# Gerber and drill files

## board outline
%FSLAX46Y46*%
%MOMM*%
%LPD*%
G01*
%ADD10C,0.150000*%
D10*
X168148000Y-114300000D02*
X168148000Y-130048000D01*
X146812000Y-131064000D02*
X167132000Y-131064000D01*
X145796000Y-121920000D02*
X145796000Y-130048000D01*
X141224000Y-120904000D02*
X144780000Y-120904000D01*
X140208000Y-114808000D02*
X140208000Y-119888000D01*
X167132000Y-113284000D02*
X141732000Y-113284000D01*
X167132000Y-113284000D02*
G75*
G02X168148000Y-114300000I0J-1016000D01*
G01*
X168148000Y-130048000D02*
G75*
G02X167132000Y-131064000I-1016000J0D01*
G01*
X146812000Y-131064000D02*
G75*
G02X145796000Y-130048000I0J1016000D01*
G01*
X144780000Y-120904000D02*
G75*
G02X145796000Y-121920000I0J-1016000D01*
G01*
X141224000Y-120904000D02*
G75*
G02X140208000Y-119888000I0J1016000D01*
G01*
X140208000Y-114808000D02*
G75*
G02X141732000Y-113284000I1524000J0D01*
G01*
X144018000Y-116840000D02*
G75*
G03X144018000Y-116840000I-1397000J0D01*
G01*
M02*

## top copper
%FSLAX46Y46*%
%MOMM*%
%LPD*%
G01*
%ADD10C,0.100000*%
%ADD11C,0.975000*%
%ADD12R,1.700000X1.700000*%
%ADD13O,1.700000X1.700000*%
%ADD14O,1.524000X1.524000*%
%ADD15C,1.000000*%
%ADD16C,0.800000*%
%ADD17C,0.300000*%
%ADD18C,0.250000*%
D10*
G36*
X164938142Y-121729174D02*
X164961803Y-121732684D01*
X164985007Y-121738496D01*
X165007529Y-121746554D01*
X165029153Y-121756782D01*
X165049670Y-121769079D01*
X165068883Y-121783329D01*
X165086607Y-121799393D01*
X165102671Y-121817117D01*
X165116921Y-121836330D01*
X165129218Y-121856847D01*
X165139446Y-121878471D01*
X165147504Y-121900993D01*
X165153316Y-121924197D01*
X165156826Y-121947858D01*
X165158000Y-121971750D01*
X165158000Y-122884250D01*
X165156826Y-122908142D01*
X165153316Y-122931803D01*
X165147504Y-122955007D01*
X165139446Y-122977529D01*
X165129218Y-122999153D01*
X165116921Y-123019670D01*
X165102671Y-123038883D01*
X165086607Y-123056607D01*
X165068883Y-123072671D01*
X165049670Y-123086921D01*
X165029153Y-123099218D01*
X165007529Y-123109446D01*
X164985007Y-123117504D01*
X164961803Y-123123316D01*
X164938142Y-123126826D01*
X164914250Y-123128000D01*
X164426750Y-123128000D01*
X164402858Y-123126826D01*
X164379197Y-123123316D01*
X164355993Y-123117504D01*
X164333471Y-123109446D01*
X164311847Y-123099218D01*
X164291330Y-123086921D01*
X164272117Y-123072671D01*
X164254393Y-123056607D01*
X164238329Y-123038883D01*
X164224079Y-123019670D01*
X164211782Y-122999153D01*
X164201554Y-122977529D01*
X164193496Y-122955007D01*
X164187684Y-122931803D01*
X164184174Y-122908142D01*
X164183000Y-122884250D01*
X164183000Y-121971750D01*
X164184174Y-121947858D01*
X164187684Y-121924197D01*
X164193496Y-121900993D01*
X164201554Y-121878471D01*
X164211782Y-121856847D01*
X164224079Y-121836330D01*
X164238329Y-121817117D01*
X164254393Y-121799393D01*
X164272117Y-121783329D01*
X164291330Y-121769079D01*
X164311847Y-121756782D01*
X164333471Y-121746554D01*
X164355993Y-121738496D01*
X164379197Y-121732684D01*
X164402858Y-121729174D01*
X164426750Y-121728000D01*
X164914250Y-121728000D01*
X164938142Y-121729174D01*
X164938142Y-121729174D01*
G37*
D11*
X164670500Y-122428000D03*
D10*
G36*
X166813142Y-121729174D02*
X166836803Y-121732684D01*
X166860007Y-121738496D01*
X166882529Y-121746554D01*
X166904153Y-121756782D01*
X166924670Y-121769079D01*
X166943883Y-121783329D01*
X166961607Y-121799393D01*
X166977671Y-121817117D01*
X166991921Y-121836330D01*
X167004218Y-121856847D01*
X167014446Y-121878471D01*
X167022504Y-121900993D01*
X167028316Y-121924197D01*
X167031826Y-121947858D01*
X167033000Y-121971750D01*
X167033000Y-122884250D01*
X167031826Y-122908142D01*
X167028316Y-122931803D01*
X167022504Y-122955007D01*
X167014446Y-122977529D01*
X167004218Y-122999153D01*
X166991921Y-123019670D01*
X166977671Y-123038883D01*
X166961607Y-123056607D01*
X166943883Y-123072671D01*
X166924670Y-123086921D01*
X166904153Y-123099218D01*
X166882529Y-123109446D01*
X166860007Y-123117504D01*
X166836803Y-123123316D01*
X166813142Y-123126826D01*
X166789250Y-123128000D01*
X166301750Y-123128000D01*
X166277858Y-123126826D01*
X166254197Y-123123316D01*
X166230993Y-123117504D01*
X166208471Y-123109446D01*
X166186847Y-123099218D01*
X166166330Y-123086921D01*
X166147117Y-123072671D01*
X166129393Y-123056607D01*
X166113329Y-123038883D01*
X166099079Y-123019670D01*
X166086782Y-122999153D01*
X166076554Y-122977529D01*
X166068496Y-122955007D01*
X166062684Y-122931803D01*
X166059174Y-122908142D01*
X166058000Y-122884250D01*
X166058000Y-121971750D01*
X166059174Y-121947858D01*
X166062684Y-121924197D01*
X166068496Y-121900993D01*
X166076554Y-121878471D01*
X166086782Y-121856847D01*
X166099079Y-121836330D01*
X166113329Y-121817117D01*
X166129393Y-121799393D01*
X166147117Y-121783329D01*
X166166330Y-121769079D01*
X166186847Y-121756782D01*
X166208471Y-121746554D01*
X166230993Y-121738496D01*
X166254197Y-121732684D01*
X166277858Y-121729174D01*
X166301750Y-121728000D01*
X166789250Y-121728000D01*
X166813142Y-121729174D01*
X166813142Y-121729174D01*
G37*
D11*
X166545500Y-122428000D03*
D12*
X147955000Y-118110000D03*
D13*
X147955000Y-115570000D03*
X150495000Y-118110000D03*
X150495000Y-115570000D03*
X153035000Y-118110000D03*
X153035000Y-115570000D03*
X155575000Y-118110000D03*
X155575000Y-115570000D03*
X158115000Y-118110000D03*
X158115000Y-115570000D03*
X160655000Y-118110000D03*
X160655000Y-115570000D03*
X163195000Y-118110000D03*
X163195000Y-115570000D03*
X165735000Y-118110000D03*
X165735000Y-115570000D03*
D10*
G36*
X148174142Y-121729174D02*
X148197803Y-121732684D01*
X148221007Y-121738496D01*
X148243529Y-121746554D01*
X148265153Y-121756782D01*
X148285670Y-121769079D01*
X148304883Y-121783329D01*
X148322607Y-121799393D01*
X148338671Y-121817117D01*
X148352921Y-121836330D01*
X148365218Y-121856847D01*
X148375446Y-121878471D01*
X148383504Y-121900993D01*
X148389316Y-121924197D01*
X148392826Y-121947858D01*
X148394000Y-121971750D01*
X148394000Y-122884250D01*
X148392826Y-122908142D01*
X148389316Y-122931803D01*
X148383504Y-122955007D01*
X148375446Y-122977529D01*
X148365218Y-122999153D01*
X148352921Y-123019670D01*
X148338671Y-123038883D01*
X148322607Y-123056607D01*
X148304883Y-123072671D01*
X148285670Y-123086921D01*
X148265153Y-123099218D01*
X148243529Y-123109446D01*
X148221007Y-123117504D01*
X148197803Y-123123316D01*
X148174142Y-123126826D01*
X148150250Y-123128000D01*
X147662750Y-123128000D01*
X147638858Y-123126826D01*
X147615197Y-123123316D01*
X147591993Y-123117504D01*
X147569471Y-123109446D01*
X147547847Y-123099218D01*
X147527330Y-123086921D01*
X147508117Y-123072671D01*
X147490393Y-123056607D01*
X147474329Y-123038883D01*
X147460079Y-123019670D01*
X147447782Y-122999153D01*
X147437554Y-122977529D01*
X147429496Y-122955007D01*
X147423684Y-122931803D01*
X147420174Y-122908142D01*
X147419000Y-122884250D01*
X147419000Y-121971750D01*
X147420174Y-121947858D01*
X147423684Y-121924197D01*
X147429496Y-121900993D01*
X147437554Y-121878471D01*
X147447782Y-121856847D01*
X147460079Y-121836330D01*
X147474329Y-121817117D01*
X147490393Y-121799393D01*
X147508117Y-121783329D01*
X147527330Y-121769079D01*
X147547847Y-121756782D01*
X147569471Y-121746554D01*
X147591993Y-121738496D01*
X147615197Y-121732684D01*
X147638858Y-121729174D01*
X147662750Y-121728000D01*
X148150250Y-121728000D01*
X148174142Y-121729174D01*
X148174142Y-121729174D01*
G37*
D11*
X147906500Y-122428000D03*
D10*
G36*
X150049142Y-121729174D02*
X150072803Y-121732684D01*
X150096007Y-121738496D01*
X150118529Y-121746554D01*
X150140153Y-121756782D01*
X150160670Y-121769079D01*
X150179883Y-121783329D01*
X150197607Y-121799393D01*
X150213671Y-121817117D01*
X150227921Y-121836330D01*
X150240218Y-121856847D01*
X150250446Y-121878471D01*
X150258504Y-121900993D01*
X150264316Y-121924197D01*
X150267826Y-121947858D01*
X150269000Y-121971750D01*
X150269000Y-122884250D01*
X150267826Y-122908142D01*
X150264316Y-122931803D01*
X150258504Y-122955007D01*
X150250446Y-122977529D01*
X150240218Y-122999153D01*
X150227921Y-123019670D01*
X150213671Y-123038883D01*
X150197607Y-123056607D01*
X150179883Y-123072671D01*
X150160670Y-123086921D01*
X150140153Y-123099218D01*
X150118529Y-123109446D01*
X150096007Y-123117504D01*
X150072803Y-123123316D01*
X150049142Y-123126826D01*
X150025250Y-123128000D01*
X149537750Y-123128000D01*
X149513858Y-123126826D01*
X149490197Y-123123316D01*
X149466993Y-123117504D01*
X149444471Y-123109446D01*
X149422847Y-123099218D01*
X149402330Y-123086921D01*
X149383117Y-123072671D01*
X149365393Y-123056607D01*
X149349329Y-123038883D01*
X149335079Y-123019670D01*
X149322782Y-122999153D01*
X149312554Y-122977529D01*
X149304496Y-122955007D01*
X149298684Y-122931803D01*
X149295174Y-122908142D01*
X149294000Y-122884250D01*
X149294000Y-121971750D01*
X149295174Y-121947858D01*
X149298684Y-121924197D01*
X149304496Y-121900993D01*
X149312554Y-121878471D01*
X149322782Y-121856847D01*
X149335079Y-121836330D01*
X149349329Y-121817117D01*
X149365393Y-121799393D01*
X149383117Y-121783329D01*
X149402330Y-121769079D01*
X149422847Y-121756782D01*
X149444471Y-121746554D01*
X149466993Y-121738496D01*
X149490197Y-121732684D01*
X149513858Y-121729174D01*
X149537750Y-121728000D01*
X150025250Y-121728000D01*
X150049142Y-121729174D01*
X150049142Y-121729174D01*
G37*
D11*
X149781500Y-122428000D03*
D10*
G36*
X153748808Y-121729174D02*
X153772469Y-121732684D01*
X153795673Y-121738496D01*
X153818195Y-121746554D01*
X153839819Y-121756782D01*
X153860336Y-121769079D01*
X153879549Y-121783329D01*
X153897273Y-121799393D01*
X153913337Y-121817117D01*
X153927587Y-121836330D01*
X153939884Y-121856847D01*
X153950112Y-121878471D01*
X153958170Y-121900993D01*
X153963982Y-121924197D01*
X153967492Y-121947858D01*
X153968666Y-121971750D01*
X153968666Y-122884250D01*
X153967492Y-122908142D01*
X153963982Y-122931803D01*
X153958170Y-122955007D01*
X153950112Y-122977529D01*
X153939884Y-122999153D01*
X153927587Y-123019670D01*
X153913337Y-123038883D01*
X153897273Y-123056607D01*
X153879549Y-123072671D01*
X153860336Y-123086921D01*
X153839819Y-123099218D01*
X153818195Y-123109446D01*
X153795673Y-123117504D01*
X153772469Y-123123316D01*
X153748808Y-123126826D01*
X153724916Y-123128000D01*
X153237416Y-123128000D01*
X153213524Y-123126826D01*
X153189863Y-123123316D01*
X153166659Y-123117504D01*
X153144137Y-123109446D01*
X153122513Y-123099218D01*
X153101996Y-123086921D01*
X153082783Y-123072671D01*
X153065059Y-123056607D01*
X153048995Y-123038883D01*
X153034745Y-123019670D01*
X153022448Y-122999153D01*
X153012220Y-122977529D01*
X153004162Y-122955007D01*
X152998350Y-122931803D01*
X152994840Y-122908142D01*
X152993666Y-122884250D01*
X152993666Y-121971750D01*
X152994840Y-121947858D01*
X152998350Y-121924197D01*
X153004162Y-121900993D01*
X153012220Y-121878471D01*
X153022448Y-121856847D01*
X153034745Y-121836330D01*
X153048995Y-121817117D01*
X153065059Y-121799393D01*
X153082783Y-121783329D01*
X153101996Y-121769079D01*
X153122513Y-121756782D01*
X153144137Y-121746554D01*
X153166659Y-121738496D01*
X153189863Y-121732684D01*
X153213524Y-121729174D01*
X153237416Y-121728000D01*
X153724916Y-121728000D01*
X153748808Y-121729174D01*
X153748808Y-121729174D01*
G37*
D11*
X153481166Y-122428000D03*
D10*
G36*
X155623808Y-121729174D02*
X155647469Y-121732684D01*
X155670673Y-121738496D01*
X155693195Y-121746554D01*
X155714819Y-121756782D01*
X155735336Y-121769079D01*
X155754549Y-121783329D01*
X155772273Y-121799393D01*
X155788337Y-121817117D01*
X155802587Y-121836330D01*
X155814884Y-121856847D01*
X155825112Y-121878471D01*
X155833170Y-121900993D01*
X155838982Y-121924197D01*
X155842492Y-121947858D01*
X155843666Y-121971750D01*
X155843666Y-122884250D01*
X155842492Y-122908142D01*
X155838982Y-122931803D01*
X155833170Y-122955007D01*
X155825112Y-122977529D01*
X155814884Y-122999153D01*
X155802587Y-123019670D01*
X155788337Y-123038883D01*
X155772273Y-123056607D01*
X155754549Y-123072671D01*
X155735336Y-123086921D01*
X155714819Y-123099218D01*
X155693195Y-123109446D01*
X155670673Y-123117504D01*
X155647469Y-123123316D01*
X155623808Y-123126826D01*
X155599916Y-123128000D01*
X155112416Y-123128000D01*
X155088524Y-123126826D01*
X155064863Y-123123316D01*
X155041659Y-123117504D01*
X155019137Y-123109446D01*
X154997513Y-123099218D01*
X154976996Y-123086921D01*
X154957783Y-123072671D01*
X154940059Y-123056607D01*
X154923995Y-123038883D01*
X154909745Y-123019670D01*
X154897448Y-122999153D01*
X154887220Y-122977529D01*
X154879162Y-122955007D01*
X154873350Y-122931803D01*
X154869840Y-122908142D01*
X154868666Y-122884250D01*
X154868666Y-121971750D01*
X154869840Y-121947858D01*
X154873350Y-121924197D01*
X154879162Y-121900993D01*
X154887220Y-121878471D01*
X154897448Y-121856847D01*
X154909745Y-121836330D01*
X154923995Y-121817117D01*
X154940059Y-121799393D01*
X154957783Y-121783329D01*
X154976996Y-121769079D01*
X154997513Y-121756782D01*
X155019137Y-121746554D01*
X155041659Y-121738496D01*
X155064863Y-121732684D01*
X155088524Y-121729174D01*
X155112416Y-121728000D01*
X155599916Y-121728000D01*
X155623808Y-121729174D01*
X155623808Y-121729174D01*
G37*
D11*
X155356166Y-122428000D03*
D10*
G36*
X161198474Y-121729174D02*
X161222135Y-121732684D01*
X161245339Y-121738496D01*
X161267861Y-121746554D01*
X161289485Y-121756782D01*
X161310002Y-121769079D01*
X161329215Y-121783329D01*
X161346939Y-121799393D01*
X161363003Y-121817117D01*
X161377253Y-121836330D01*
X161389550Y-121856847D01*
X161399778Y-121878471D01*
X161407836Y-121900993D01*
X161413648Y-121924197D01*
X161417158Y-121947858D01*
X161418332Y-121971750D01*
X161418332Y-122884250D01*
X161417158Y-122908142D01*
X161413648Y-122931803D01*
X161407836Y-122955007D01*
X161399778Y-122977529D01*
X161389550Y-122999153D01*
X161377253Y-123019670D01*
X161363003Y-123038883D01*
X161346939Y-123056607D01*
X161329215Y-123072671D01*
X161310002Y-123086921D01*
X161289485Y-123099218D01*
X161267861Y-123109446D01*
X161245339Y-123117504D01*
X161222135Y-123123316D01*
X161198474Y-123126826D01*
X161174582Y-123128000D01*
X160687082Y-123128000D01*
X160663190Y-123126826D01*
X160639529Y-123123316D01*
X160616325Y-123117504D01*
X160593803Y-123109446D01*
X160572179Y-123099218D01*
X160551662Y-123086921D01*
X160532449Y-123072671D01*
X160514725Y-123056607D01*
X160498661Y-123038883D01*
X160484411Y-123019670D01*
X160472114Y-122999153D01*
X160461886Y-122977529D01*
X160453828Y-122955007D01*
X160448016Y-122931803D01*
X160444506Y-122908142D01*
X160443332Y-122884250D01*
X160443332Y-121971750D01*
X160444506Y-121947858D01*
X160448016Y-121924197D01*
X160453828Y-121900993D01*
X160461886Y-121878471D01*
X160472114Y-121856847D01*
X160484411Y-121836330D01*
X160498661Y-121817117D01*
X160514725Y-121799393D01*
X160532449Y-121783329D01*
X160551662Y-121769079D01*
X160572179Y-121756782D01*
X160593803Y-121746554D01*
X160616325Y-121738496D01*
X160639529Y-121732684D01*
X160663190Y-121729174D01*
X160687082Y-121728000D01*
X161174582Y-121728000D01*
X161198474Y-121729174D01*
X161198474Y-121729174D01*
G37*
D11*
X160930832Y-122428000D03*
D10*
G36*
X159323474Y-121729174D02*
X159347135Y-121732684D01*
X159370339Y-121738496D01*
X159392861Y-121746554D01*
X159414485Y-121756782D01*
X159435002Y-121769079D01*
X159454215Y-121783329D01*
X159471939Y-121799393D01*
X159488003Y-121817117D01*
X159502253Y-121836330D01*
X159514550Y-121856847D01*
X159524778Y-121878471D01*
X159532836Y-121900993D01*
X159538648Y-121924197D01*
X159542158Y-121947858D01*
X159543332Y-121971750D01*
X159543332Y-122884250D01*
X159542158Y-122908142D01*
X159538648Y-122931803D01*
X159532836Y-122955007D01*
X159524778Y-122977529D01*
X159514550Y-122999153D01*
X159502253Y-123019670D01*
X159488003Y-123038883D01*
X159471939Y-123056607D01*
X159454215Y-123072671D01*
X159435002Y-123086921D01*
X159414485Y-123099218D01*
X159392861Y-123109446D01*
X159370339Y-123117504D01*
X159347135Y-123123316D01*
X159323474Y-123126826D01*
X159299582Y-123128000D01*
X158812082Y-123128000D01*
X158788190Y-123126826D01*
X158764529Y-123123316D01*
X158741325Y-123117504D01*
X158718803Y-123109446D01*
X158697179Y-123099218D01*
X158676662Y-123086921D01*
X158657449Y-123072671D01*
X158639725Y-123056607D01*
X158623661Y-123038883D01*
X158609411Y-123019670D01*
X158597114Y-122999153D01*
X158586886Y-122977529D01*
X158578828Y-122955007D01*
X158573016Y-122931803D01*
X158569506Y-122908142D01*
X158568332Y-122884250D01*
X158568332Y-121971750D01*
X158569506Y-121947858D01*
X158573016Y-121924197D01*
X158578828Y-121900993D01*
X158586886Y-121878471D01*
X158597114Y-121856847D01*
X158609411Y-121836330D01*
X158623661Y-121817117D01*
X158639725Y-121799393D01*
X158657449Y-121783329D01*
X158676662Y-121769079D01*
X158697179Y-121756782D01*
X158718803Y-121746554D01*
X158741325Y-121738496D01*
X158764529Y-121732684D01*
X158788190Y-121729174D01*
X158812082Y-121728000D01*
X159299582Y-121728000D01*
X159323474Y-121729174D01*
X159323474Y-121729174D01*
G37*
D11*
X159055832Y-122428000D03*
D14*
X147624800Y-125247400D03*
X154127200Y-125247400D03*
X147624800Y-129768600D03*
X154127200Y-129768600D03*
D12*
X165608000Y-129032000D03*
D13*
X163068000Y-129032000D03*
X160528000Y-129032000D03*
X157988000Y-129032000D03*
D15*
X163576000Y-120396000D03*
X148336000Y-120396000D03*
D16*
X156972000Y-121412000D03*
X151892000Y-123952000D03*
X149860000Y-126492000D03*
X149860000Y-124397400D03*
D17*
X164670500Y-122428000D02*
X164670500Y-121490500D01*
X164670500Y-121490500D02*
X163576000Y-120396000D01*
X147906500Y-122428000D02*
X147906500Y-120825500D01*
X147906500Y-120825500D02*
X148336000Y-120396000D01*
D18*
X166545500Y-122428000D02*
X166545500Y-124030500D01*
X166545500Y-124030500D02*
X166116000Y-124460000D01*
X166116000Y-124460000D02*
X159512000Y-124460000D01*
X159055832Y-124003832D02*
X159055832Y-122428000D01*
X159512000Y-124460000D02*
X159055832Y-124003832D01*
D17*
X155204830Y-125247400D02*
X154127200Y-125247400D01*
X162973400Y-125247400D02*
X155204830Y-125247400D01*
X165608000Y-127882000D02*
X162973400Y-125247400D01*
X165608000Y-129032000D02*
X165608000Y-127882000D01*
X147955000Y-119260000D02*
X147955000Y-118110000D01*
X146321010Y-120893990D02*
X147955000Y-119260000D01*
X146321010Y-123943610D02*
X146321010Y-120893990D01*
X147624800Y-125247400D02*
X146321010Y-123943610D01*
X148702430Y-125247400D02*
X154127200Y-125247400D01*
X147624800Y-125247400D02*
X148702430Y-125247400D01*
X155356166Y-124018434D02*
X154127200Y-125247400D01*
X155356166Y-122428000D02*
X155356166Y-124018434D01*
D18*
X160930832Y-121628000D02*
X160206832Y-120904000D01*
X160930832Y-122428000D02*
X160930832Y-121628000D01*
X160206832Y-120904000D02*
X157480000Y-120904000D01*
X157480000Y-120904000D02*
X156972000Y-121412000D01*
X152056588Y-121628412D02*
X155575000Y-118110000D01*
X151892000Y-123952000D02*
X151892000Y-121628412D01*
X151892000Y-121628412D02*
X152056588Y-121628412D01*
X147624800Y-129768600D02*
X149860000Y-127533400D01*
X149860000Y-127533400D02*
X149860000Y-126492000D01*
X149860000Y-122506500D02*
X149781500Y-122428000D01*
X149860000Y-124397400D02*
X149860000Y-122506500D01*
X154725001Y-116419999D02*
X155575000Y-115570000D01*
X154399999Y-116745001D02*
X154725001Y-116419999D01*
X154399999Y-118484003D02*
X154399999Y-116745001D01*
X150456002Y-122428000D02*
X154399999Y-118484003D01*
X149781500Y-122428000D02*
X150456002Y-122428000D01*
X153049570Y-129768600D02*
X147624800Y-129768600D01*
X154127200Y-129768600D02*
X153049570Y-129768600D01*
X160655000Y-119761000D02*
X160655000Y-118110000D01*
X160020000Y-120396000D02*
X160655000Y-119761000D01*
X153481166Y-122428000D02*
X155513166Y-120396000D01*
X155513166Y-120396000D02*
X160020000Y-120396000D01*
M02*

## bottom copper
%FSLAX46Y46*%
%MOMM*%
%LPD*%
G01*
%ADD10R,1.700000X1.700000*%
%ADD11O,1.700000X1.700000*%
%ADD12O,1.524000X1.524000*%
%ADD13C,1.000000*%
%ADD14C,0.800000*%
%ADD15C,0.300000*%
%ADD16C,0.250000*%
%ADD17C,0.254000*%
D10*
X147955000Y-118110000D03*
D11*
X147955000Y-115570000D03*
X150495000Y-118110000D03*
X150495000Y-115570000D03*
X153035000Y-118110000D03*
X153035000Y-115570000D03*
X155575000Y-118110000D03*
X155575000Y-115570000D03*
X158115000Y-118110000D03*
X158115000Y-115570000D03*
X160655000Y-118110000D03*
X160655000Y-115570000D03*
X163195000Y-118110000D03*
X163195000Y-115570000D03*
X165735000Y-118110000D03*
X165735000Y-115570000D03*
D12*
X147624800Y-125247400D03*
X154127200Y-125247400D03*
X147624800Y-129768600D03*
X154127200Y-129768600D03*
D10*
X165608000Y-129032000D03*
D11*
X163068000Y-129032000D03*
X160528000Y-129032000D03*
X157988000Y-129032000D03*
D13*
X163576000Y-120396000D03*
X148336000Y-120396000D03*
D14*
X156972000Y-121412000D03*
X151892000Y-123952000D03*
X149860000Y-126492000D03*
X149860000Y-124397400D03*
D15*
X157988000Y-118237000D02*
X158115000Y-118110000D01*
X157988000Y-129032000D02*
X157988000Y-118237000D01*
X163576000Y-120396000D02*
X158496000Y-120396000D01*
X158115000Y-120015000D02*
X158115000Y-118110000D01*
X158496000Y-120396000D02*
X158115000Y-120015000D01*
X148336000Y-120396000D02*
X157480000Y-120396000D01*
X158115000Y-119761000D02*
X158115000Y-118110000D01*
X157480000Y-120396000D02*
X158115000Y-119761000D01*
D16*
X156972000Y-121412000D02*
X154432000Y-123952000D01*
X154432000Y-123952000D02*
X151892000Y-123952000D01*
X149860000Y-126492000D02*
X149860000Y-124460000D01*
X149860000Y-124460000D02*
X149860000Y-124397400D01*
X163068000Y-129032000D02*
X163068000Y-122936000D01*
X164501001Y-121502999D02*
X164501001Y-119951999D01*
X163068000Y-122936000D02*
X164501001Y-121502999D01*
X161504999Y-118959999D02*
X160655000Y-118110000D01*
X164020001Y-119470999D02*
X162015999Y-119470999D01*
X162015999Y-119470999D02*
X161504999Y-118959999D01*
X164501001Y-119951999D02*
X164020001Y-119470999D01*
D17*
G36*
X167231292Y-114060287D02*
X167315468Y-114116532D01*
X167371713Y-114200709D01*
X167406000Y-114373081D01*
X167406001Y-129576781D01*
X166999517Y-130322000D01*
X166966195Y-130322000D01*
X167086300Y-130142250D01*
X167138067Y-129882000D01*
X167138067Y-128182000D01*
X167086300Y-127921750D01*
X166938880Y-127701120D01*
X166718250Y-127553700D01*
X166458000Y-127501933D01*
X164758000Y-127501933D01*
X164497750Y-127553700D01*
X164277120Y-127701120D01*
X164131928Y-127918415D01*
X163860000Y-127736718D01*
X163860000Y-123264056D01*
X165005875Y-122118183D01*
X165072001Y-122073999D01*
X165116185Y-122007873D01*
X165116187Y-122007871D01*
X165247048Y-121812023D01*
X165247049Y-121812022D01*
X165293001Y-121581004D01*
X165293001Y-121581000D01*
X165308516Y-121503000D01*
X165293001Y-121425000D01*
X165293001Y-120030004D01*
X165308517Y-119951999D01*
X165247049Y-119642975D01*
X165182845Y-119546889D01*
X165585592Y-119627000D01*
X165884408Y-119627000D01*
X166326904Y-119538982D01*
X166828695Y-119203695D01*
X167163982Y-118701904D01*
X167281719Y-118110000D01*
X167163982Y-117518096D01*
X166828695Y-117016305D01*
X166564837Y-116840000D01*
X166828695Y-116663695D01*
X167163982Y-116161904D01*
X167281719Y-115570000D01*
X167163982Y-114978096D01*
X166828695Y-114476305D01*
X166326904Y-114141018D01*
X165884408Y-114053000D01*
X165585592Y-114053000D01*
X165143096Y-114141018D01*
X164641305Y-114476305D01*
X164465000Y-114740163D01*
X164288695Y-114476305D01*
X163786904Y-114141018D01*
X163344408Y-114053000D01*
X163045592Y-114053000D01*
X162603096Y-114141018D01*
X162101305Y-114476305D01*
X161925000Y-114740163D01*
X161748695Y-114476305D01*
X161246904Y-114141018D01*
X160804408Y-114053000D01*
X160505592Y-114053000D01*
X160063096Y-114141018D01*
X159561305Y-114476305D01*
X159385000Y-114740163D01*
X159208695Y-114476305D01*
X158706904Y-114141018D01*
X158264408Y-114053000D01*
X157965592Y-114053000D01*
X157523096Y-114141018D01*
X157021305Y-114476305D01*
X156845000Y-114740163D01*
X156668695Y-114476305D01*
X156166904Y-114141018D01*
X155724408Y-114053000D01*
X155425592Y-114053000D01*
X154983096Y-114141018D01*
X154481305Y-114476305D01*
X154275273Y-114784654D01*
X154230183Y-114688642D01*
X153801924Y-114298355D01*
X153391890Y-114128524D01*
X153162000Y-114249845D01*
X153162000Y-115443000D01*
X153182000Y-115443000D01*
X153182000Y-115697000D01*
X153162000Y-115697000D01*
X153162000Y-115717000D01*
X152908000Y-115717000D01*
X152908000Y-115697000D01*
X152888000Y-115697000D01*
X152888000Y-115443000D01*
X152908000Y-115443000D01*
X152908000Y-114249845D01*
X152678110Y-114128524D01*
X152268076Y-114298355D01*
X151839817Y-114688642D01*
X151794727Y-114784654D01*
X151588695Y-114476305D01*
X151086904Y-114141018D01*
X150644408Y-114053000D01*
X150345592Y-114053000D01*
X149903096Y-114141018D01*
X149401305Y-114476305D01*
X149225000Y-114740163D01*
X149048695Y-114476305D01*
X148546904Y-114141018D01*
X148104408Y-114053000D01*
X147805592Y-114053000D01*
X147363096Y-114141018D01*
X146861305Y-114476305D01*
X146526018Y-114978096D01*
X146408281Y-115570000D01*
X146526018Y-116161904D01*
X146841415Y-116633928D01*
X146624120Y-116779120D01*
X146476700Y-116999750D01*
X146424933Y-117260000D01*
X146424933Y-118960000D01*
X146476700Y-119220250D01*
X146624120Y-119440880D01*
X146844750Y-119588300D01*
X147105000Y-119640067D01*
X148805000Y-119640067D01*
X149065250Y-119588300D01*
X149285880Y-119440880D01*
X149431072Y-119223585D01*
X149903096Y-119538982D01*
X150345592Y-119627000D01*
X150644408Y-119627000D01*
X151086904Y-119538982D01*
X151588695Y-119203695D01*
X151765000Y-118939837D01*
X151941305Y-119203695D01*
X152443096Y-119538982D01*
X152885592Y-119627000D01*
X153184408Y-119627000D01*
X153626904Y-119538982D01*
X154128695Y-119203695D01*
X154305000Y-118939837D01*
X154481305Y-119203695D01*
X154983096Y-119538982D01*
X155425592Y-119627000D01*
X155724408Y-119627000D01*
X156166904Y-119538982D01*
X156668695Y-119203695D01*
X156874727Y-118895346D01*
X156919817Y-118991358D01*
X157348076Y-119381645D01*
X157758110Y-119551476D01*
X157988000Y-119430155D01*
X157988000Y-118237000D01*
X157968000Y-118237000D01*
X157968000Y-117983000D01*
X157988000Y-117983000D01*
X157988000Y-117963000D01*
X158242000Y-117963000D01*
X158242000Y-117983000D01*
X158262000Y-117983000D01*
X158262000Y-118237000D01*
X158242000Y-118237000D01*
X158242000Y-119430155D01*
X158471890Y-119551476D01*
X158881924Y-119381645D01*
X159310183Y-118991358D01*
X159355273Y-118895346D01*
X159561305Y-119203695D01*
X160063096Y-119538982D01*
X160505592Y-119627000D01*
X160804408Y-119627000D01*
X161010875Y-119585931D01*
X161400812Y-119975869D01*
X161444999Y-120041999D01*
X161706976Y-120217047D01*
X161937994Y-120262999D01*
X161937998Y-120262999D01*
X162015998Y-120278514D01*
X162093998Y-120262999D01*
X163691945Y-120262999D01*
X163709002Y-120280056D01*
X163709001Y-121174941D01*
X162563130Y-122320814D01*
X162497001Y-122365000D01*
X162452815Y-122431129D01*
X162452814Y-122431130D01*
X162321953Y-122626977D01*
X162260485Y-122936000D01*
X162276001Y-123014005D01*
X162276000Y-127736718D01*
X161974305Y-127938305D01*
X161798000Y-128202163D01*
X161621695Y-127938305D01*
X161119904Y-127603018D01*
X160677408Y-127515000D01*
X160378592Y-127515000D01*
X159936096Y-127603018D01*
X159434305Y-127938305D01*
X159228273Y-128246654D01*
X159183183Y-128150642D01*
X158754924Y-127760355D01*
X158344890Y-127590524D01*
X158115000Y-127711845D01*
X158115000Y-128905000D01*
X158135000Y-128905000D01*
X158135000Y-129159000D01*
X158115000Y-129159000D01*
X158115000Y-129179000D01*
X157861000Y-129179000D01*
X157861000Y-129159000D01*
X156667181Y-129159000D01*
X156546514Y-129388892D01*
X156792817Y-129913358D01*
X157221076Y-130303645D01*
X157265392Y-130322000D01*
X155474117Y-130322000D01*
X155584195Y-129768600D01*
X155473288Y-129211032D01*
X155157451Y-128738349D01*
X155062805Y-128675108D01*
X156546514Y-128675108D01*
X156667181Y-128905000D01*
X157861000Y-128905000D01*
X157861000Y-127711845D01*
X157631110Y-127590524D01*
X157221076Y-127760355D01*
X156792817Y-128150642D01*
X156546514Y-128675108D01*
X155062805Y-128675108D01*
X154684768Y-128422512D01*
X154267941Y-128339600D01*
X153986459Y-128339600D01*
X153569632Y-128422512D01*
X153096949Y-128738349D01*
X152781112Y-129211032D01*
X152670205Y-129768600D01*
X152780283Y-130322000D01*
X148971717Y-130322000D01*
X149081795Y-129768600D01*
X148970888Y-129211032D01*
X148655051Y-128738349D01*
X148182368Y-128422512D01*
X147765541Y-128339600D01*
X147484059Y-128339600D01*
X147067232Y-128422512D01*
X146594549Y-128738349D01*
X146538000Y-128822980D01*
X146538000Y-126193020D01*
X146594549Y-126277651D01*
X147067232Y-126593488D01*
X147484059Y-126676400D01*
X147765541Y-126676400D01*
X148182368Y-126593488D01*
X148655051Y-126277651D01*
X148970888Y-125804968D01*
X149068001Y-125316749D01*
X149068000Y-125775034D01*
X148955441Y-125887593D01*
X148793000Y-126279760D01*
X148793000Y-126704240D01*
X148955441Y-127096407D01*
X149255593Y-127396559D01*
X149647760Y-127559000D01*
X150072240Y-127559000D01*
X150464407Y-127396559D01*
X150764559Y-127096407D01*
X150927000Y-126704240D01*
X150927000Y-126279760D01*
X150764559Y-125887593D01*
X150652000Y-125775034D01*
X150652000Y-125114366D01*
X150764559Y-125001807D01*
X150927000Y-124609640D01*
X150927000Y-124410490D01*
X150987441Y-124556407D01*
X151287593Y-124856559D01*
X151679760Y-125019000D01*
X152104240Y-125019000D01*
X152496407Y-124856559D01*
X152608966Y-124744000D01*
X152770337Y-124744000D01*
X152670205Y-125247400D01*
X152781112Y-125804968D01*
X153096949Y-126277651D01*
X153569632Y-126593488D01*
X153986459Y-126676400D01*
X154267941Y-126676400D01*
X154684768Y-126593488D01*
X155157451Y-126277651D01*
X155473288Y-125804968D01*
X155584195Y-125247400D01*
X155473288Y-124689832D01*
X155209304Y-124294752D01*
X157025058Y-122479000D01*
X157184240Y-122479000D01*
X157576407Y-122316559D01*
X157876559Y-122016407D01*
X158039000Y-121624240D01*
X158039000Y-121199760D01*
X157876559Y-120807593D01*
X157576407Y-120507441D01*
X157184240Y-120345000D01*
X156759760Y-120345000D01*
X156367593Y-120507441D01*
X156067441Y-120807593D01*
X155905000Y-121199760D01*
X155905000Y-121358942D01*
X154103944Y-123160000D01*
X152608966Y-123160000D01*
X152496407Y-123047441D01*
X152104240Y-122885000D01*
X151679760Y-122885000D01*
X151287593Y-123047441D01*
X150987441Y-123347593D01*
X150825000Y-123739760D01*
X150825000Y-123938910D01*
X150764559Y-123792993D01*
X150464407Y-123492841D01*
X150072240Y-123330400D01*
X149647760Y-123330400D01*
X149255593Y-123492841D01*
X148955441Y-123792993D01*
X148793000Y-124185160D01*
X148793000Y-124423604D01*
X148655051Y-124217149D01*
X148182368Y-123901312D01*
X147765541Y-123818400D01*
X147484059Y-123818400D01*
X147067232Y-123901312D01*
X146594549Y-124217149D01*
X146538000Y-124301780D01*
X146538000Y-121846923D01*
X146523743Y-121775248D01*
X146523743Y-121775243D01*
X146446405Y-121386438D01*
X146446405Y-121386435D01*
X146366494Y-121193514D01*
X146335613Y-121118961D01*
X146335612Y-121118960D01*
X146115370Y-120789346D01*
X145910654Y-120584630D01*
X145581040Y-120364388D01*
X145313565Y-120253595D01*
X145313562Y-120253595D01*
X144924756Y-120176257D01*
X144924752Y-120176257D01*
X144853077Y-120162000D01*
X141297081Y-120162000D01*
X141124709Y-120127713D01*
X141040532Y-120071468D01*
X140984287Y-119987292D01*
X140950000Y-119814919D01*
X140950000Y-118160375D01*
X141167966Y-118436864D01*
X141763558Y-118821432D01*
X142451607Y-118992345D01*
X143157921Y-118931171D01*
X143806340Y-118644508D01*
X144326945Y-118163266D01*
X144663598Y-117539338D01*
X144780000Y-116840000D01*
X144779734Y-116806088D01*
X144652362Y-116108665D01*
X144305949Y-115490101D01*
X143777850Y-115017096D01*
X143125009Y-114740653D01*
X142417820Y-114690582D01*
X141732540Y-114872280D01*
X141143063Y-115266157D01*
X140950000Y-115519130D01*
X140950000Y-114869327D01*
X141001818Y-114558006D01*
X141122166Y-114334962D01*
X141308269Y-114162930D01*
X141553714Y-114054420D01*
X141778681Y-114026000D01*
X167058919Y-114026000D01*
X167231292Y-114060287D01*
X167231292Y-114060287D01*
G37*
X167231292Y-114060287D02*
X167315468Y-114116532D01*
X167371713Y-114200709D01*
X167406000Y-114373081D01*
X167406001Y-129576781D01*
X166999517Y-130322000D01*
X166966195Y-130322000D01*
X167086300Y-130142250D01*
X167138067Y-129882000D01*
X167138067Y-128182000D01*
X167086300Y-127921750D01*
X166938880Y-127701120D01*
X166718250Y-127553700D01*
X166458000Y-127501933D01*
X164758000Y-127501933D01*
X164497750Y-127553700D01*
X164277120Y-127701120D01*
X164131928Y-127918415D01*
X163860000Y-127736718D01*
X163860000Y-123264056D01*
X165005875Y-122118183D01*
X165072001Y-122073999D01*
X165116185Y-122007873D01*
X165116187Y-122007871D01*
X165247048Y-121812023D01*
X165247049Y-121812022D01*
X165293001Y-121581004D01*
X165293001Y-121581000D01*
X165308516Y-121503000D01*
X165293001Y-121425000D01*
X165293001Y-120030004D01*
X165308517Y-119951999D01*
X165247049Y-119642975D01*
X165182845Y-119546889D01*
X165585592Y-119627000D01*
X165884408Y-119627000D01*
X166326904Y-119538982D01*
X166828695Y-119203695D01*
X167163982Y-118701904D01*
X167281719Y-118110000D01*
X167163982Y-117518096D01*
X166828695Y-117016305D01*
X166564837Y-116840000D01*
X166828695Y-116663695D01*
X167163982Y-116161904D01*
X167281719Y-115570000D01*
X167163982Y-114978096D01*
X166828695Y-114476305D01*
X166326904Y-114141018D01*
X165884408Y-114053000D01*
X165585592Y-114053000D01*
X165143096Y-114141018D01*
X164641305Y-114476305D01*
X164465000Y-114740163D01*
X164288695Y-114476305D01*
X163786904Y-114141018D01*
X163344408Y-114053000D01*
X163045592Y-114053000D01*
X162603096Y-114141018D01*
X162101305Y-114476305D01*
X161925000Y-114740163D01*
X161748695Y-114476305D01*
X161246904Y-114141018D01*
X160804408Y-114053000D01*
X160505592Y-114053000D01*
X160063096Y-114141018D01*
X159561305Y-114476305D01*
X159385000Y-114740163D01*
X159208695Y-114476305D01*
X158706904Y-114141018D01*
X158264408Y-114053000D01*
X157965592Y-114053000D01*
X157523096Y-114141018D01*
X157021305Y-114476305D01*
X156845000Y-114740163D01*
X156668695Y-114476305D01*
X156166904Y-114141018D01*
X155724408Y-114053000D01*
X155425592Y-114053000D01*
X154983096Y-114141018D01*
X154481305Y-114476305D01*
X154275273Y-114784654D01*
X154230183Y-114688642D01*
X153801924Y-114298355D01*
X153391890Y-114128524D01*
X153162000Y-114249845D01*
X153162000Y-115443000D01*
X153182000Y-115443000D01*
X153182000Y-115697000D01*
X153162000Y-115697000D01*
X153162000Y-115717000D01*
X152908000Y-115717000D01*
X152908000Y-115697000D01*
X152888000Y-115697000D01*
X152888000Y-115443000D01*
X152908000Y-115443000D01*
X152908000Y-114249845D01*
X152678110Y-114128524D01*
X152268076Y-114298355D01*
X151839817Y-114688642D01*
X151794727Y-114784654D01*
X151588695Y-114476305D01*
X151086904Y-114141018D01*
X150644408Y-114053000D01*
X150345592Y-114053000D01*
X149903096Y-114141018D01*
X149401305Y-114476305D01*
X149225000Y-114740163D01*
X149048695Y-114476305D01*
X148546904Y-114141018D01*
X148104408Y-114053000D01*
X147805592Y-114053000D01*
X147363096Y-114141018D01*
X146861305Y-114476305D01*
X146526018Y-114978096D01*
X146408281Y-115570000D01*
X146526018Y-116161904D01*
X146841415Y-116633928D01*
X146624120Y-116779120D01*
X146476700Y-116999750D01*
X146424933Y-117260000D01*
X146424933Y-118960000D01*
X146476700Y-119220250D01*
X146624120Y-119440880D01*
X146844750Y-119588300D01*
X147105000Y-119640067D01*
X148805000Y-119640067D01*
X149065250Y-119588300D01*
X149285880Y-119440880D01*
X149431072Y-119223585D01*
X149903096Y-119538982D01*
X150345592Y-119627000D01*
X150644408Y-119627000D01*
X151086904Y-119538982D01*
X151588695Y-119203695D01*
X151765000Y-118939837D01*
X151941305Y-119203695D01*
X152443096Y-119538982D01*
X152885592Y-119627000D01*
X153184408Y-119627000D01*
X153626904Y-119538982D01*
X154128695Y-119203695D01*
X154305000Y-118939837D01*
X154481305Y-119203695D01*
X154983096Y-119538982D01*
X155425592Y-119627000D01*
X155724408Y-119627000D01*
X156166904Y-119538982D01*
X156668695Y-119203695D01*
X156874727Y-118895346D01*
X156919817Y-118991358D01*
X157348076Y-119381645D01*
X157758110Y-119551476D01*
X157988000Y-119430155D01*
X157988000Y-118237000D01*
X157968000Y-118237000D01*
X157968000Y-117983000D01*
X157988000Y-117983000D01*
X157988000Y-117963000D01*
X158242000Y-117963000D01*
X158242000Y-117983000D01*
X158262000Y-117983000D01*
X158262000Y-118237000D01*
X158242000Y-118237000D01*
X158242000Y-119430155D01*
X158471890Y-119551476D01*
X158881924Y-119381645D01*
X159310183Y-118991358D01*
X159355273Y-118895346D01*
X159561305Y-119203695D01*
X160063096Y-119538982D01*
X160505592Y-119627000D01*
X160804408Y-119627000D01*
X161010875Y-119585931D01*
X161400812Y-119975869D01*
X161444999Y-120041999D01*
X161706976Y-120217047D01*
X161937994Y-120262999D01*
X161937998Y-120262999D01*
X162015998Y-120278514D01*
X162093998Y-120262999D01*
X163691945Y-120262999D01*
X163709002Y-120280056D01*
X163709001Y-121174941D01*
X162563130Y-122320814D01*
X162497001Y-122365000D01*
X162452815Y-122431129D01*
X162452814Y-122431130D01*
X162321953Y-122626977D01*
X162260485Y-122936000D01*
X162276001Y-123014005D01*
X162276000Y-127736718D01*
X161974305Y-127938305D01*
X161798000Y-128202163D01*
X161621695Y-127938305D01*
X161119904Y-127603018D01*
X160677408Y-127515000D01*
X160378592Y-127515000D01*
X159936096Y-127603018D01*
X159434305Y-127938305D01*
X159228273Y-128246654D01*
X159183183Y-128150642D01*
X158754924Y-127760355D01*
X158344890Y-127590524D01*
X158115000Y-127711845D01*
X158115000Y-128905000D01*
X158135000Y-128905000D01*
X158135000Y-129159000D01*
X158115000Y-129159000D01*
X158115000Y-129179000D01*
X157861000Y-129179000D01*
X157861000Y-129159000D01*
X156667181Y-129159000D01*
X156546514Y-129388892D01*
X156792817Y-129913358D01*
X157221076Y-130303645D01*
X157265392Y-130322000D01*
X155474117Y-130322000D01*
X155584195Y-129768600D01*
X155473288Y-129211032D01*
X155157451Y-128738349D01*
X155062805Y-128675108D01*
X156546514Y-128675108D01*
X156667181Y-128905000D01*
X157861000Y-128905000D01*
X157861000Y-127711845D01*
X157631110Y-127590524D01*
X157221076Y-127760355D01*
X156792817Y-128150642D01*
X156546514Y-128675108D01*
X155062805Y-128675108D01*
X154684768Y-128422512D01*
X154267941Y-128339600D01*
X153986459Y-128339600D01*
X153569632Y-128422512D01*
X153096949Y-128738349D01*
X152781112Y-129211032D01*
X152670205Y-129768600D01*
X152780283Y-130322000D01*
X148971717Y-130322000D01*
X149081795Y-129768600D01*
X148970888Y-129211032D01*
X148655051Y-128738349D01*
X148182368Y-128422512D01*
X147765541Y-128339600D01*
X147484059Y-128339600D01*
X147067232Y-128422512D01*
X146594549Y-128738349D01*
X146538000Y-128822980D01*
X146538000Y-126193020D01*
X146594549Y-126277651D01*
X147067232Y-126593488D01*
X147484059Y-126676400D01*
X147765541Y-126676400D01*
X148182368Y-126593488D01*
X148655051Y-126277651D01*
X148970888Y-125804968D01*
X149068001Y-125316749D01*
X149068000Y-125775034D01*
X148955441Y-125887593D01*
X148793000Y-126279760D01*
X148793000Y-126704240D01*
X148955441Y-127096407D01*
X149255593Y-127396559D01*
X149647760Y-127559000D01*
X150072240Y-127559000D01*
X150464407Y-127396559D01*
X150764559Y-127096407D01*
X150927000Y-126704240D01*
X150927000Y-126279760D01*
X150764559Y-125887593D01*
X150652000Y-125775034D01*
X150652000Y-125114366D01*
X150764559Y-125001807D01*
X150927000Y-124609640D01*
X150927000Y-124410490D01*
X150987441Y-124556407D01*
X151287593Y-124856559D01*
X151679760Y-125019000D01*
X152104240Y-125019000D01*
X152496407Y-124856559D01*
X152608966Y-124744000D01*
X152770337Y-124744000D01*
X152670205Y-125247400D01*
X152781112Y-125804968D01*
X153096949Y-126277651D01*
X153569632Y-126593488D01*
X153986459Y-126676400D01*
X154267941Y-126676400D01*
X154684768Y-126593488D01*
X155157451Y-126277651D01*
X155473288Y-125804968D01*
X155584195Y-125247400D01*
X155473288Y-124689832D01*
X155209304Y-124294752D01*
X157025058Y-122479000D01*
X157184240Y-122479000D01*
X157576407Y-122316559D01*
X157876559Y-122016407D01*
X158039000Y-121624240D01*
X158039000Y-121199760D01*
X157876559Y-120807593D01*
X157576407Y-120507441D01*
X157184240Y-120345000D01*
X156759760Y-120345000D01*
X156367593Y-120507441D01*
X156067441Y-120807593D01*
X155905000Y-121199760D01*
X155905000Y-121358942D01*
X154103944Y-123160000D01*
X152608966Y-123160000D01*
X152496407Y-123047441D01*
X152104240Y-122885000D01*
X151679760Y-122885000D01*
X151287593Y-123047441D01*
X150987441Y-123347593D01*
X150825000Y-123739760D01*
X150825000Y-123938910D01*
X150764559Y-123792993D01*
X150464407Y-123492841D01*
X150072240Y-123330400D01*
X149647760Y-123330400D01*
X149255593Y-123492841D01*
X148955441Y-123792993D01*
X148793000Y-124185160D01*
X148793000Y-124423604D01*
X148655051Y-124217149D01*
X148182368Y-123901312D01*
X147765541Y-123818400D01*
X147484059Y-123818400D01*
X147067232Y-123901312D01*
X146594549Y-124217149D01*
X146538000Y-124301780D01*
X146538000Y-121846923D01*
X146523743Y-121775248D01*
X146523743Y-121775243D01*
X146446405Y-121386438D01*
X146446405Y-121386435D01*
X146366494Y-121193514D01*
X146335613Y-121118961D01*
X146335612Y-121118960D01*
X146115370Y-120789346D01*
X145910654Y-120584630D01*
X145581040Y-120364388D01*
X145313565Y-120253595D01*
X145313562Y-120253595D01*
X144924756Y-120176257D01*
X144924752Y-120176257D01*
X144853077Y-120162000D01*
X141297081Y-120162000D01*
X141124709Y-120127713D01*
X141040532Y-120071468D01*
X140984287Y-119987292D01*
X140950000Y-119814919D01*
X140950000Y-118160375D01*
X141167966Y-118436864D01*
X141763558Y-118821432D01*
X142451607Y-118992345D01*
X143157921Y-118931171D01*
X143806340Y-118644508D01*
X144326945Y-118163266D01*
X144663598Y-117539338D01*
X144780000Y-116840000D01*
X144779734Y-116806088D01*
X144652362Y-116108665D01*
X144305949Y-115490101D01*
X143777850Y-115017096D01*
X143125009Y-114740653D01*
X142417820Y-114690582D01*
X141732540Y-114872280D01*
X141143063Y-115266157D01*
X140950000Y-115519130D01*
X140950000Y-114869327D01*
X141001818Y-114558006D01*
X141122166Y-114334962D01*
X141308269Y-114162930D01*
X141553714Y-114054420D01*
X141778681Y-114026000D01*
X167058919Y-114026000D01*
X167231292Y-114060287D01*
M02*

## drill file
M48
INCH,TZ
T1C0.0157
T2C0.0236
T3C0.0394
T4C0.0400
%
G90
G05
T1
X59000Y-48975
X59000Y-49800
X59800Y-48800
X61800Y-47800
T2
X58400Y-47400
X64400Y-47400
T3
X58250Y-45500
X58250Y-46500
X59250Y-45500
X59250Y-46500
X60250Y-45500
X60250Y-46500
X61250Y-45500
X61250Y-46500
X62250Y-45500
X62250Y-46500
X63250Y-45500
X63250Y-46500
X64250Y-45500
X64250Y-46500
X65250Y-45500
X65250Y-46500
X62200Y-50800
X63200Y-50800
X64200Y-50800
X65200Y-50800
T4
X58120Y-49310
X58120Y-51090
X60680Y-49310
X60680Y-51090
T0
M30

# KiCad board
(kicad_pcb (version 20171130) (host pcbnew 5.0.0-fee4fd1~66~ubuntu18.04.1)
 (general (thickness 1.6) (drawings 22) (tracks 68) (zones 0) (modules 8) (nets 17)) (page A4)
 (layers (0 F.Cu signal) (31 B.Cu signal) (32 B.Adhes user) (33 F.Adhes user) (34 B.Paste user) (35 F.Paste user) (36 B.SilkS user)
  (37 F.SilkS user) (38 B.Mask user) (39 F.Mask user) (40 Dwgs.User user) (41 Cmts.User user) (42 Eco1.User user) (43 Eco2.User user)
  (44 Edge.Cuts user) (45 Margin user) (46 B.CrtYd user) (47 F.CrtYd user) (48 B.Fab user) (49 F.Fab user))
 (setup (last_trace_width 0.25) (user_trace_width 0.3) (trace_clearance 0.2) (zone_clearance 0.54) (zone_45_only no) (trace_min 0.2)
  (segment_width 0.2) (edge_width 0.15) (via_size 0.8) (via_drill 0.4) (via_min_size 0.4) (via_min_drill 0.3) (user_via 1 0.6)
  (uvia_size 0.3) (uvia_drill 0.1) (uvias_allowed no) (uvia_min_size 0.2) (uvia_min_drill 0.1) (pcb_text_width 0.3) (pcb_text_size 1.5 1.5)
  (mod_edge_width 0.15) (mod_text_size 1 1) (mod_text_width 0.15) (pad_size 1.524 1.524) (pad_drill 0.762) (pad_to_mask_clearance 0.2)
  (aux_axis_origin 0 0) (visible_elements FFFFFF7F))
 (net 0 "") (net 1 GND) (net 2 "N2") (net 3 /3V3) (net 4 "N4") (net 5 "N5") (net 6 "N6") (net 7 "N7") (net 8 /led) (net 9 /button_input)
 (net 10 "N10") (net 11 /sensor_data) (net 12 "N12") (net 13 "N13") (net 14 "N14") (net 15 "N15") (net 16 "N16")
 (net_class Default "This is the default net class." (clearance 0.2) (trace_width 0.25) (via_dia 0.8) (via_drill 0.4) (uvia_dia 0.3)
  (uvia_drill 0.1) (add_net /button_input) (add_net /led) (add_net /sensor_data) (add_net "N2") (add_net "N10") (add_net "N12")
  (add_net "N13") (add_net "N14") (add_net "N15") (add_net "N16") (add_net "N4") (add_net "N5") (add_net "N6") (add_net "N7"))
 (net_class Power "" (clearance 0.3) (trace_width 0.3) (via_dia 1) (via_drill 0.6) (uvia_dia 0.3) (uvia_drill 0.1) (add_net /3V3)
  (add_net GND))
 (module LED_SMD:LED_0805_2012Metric (layer F.Cu) (at 165.608 122.428)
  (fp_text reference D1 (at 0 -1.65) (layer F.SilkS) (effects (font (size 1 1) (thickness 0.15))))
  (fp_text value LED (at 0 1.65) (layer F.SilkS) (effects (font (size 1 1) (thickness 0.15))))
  (pad 1 smd roundrect (at -0.9375 0) (size 0.975 1.4) (layers F.Cu F.Paste F.Mask) (roundrect_rratio 0.25) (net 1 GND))
  (pad 2 smd roundrect (at 0.9375 0) (size 0.975 1.4) (layers F.Cu F.Paste F.Mask) (roundrect_rratio 0.25) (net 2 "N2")))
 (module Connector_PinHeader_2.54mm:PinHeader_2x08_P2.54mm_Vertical (layer F.Cu) (at 147.955 118.11 90)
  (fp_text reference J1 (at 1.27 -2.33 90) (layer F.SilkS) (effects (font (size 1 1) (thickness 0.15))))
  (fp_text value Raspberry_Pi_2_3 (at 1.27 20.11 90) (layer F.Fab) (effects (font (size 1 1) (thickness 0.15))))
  (pad 1 thru_hole rect (at 0 0 90) (size 1.7 1.7) (drill 1) (layers *.Cu *.Mask) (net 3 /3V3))
  (pad 2 thru_hole oval (at 2.54 0 90) (size 1.7 1.7) (drill 1) (layers *.Cu *.Mask) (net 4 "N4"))
  (pad 3 thru_hole oval (at 0 2.54 90) (size 1.7 1.7) (drill 1) (layers *.Cu *.Mask) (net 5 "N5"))
  (pad 4 thru_hole oval (at 2.54 2.54 90) (size 1.7 1.7) (drill 1) (layers *.Cu *.Mask) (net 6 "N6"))
  (pad 5 thru_hole oval (at 0 5.08 90) (size 1.7 1.7) (drill 1) (layers *.Cu *.Mask) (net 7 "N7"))
  (pad 6 thru_hole oval (at 2.54 5.08 90) (size 1.7 1.7) (drill 1) (layers *.Cu *.Mask) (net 1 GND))
  (pad 7 thru_hole oval (at 0 7.62 90) (size 1.7 1.7) (drill 1) (layers *.Cu *.Mask) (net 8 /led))
  (pad 8 thru_hole oval (at 2.54 7.62 90) (size 1.7 1.7) (drill 1) (layers *.Cu *.Mask) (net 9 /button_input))
  (pad 9 thru_hole oval (at 0 10.16 90) (size 1.7 1.7) (drill 1) (layers *.Cu *.Mask) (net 1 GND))
  (pad 10 thru_hole oval (at 2.54 10.16 90) (size 1.7 1.7) (drill 1) (layers *.Cu *.Mask) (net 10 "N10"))
  (pad 11 thru_hole oval (at 0 12.7 90) (size 1.7 1.7) (drill 1) (layers *.Cu *.Mask) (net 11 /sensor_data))
  (pad 12 thru_hole oval (at 2.54 12.7 90) (size 1.7 1.7) (drill 1) (layers *.Cu *.Mask) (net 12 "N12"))
  (pad 13 thru_hole oval (at 0 15.24 90) (size 1.7 1.7) (drill 1) (layers *.Cu *.Mask) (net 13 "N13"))
  (pad 14 thru_hole oval (at 2.54 15.24 90) (size 1.7 1.7) (drill 1) (layers *.Cu *.Mask) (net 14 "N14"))
  (pad 15 thru_hole oval (at 0 17.78 90) (size 1.7 1.7) (drill 1) (layers *.Cu *.Mask) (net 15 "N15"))
  (pad 16 thru_hole oval (at 2.54 17.78 90) (size 1.7 1.7) (drill 1) (layers *.Cu *.Mask) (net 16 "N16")))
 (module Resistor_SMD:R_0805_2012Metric (layer F.Cu) (at 148.844 122.428)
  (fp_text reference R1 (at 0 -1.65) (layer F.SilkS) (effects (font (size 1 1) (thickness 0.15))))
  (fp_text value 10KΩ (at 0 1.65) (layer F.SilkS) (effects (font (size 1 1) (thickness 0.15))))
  (pad 1 smd roundrect (at -0.9375 0) (size 0.975 1.4) (layers F.Cu F.Paste F.Mask) (roundrect_rratio 0.25) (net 1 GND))
  (pad 2 smd roundrect (at 0.9375 0) (size 0.975 1.4) (layers F.Cu F.Paste F.Mask) (roundrect_rratio 0.25) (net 9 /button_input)))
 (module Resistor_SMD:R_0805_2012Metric (layer F.Cu) (at 154.418666 122.428)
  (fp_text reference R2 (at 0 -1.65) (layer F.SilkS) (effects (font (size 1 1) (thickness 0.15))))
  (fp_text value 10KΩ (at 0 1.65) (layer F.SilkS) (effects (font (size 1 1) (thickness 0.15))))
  (pad 1 smd roundrect (at -0.9375 0) (size 0.975 1.4) (layers F.Cu F.Paste F.Mask) (roundrect_rratio 0.25) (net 11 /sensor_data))
  (pad 2 smd roundrect (at 0.9375 0) (size 0.975 1.4) (layers F.Cu F.Paste F.Mask) (roundrect_rratio 0.25) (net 3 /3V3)))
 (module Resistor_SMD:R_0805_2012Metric (layer F.Cu) (at 159.993332 122.428)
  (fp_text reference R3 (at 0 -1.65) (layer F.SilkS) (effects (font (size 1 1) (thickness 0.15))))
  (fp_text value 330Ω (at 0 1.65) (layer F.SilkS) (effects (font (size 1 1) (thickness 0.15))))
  (pad 2 smd roundrect (at 0.9375 0) (size 0.975 1.4) (layers F.Cu F.Paste F.Mask) (roundrect_rratio 0.25) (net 8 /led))
  (pad 1 smd roundrect (at -0.9375 0) (size 0.975 1.4) (layers F.Cu F.Paste F.Mask) (roundrect_rratio 0.25) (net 2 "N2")))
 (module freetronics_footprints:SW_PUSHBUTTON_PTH (layer F.Cu) (at 150.876 127.508)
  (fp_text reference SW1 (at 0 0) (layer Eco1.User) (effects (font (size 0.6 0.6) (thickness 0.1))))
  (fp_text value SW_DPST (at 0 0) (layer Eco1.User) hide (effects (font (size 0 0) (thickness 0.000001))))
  (pad 1 thru_hole oval (at -3.2512 -2.2606) (size 1.524 1.524) (drill 1.016) (layers *.Cu *.Mask) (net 3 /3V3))
  (pad 1 thru_hole oval (at 3.2512 -2.2606) (size 1.524 1.524) (drill 1.016) (layers *.Cu *.Mask) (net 3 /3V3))
  (pad 2 thru_hole oval (at -3.2512 2.2606) (size 1.524 1.524) (drill 1.016) (layers *.Cu *.Mask) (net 9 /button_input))
  (pad 2 thru_hole oval (at 3.2512 2.2606) (size 1.524 1.524) (drill 1.016) (layers *.Cu *.Mask) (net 9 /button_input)))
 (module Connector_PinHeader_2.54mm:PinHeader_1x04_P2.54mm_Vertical (layer F.Cu) (at 165.608 129.032 270)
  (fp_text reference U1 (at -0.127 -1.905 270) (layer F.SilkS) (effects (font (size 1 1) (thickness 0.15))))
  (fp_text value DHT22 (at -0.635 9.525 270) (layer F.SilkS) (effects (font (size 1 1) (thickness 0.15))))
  (pad 1 thru_hole rect (at 0 0 270) (size 1.7 1.7) (drill 1) (layers *.Cu *.Mask) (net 3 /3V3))
  (pad 2 thru_hole oval (at 0 2.54 270) (size 1.7 1.7) (drill 1) (layers *.Cu *.Mask) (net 11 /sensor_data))
  (pad 3 thru_hole oval (at 0 5.08 270) (size 1.7 1.7) (drill 1) (layers *.Cu *.Mask))
  (pad 4 thru_hole oval (at 0 7.62 270) (size 1.7 1.7) (drill 1) (layers *.Cu *.Mask) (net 1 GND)))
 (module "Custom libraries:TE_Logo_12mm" (layer B.Cu) (at 152.654 121.666 180)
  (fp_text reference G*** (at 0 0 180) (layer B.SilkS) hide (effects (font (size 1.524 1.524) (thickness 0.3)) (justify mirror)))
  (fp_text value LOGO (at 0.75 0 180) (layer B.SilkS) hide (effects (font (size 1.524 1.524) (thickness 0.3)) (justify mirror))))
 (gr_line (start 168.148 114.3) (end 168.148 130.048) (layer Edge.Cuts) (width 0.15))
 (gr_line (start 146.812 131.064) (end 167.132 131.064) (layer Edge.Cuts) (width 0.15))
 (gr_line (start 145.796 121.92) (end 145.796 130.048) (layer Edge.Cuts) (width 0.15))
 (gr_line (start 141.224 120.904) (end 144.78 120.904) (layer Edge.Cuts) (width 0.15))
 (gr_line (start 140.208 114.808) (end 140.208 119.888) (layer Edge.Cuts) (width 0.15))
 (gr_line (start 167.132 113.284) (end 141.732 113.284) (layer Edge.Cuts) (width 0.15))
 (gr_arc (start 167.132 114.3) (end 168.148 114.3) (angle -90) (layer Edge.Cuts) (width 0.15))
 (gr_arc (start 167.132 130.048) (end 167.132 131.064) (angle -90) (layer Edge.Cuts) (width 0.15))
 (gr_arc (start 146.812 130.048) (end 145.796 130.048) (angle -90) (layer Edge.Cuts) (width 0.15))
 (gr_arc (start 144.78 121.92) (end 145.796 121.92) (angle -90) (layer Edge.Cuts) (width 0.15))
 (gr_arc (start 141.224 119.888) (end 140.208 119.888) (angle -90) (layer Edge.Cuts) (width 0.15))
 (gr_arc (start 141.732 114.808) (end 141.732 113.284) (angle -90) (layer Edge.Cuts) (width 0.15))
 (gr_circle (center 142.621 116.84) (end 141.224 116.84) (layer Edge.Cuts) (width 0.15))
 (segment (start 157.988 118.237) (end 158.115 118.11) (width 0.3) (layer B.Cu) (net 1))
 (segment (start 157.988 129.032) (end 157.988 118.237) (width 0.3) (layer B.Cu) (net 1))
 (via (at 163.576 120.396) (size 1) (drill 0.6) (layers F.Cu B.Cu) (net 1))
 (segment (start 164.6705 122.428) (end 164.6705 121.4905) (width 0.3) (layer F.Cu) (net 1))
 (segment (start 164.6705 121.4905) (end 163.576 120.396) (width 0.3) (layer F.Cu) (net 1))
 (segment (start 163.576 120.396) (end 158.496 120.396) (width 0.3) (layer B.Cu) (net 1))
 (segment (start 158.115 120.015) (end 158.115 118.11) (width 0.3) (layer B.Cu) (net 1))
 (segment (start 158.496 120.396) (end 158.115 120.015) (width 0.3) (layer B.Cu) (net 1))
 (via (at 148.336 120.396) (size 1) (drill 0.6) (layers F.Cu B.Cu) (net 1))
 (segment (start 147.9065 122.428) (end 147.9065 120.8255) (width 0.3) (layer F.Cu) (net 1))
 (segment (start 147.9065 120.8255) (end 148.336 120.396) (width 0.3) (layer F.Cu) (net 1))
 (segment (start 148.336 120.396) (end 157.48 120.396) (width 0.3) (layer B.Cu) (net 1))
 (segment (start 158.115 119.761) (end 158.115 118.11) (width 0.3) (layer B.Cu) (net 1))
 (segment (start 157.48 120.396) (end 158.115 119.761) (width 0.3) (layer B.Cu) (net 1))
 (segment (start 166.5455 122.428) (end 166.5455 124.0305) (width 0.25) (layer F.Cu) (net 2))
 (segment (start 166.5455 124.0305) (end 166.116 124.46) (width 0.25) (layer F.Cu) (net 2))
 (segment (start 166.116 124.46) (end 159.512 124.46) (width 0.25) (layer F.Cu) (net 2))
 (segment (start 159.055832 124.003832) (end 159.055832 122.428) (width 0.25) (layer F.Cu) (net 2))
 (segment (start 159.512 124.46) (end 159.055832 124.003832) (width 0.25) (layer F.Cu) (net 2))
 (segment (start 155.20483 125.2474) (end 154.1272 125.2474) (width 0.3) (layer F.Cu) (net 3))
 (segment (start 162.9734 125.2474) (end 155.20483 125.2474) (width 0.3) (layer F.Cu) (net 3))
 (segment (start 165.608 127.882) (end 162.9734 125.2474) (width 0.3) (layer F.Cu) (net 3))
 (segment (start 165.608 129.032) (end 165.608 127.882) (width 0.3) (layer F.Cu) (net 3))
 (segment (start 147.955 119.26) (end 147.955 118.11) (width 0.3) (layer F.Cu) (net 3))
 (segment (start 146.32101 120.89399) (end 147.955 119.26) (width 0.3) (layer F.Cu) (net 3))
 (segment (start 146.32101 123.94361) (end 146.32101 120.89399) (width 0.3) (layer F.Cu) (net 3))
 (segment (start 147.6248 125.2474) (end 146.32101 123.94361) (width 0.3) (layer F.Cu) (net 3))
 (segment (start 148.70243 125.2474) (end 154.1272 125.2474) (width 0.3) (layer F.Cu) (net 3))
 (segment (start 147.6248 125.2474) (end 148.70243 125.2474) (width 0.3) (layer F.Cu) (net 3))
 (segment (start 155.356166 124.018434) (end 154.1272 125.2474) (width 0.3) (layer F.Cu) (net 3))
 (segment (start 155.356166 122.428) (end 155.356166 124.018434) (width 0.3) (layer F.Cu) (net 3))
 (segment (start 160.930832 121.628) (end 160.206832 120.904) (width 0.25) (layer F.Cu) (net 8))
 (segment (start 160.930832 122.428) (end 160.930832 121.628) (width 0.25) (layer F.Cu) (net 8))
 (via (at 156.972 121.412) (size 0.8) (drill 0.4) (layers F.Cu B.Cu) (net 8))
 (segment (start 160.206832 120.904) (end 157.48 120.904) (width 0.25) (layer F.Cu) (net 8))
 (segment (start 157.48 120.904) (end 156.972 121.412) (width 0.25) (layer F.Cu) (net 8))
 (via (at 151.892 123.952) (size 0.8) (drill 0.4) (layers F.Cu B.Cu) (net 8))
 (segment (start 156.972 121.412) (end 154.432 123.952) (width 0.25) (layer B.Cu) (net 8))
 (segment (start 154.432 123.952) (end 151.892 123.952) (width 0.25) (layer B.Cu) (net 8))
 (segment (start 152.056588 121.628412) (end 155.575 118.11) (width 0.25) (layer F.Cu) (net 8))
 (segment (start 151.892 123.952) (end 151.892 121.628412) (width 0.25) (layer F.Cu) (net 8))
 (segment (start 151.892 121.628412) (end 152.056588 121.628412) (width 0.25) (layer F.Cu) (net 8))
 (via (at 149.86 126.492) (size 0.8) (drill 0.4) (layers F.Cu B.Cu) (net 9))
 (segment (start 147.6248 129.7686) (end 149.86 127.5334) (width 0.25) (layer F.Cu) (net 9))
 (segment (start 149.86 127.5334) (end 149.86 126.492) (width 0.25) (layer F.Cu) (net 9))
 (segment (start 149.86 126.492) (end 149.86 124.46) (width 0.25) (layer B.Cu) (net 9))
 (via (at 149.86 124.3974) (size 0.8) (drill 0.4) (layers F.Cu B.Cu) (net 9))
 (segment (start 149.86 124.46) (end 149.86 124.3974) (width 0.25) (layer B.Cu) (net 9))
 (segment (start 149.86 122.5065) (end 149.7815 122.428) (width 0.25) (layer F.Cu) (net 9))
 (segment (start 149.86 124.3974) (end 149.86 122.5065) (width 0.25) (layer F.Cu) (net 9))
 (segment (start 154.725001 116.419999) (end 155.575 115.57) (width 0.25) (layer F.Cu) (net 9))
 (segment (start 154.399999 116.745001) (end 154.725001 116.419999) (width 0.25) (layer F.Cu) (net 9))
 (segment (start 154.399999 118.484003) (end 154.399999 116.745001) (width 0.25) (layer F.Cu) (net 9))
 (segment (start 150.456002 122.428) (end 154.399999 118.484003) (width 0.25) (layer F.Cu) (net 9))
 (segment (start 149.7815 122.428) (end 150.456002 122.428) (width 0.25) (layer F.Cu) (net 9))
 (segment (start 153.04957 129.7686) (end 147.6248 129.7686) (width 0.25) (layer F.Cu) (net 9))
 (segment (start 154.1272 129.7686) (end 153.04957 129.7686) (width 0.25) (layer F.Cu) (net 9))
 (segment (start 160.655 119.761) (end 160.655 118.11) (width 0.25) (layer F.Cu) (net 11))
 (segment (start 160.02 120.396) (end 160.655 119.761) (width 0.25) (layer F.Cu) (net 11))
 (segment (start 153.481166 122.428) (end 155.513166 120.396) (width 0.25) (layer F.Cu) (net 11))
 (segment (start 155.513166 120.396) (end 160.02 120.396) (width 0.25) (layer F.Cu) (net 11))
 (segment (start 163.068 129.032) (end 163.068 122.936) (width 0.25) (layer B.Cu) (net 11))
 (segment (start 164.501001 121.502999) (end 164.501001 119.951999) (width 0.25) (layer B.Cu) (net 11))
 (segment (start 163.068 122.936) (end 164.501001 121.502999) (width 0.25) (layer B.Cu) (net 11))
 (segment (start 161.504999 118.959999) (end 160.655 118.11) (width 0.25) (layer B.Cu) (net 11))
 (segment (start 164.020001 119.470999) (end 162.015999 119.470999) (width 0.25) (layer B.Cu) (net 11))
 (segment (start 162.015999 119.470999) (end 161.504999 118.959999) (width 0.25) (layer B.Cu) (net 11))
 (segment (start 164.501001 119.951999) (end 164.020001 119.470999) (width 0.25) (layer B.Cu) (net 11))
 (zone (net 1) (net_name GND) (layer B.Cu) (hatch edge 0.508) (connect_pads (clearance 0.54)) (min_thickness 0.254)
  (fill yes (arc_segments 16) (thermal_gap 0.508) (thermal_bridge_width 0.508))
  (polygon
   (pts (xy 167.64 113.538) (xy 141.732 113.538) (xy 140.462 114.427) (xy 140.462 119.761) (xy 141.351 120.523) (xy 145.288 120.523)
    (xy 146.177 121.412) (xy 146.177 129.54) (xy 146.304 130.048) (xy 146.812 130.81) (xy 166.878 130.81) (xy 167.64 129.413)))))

